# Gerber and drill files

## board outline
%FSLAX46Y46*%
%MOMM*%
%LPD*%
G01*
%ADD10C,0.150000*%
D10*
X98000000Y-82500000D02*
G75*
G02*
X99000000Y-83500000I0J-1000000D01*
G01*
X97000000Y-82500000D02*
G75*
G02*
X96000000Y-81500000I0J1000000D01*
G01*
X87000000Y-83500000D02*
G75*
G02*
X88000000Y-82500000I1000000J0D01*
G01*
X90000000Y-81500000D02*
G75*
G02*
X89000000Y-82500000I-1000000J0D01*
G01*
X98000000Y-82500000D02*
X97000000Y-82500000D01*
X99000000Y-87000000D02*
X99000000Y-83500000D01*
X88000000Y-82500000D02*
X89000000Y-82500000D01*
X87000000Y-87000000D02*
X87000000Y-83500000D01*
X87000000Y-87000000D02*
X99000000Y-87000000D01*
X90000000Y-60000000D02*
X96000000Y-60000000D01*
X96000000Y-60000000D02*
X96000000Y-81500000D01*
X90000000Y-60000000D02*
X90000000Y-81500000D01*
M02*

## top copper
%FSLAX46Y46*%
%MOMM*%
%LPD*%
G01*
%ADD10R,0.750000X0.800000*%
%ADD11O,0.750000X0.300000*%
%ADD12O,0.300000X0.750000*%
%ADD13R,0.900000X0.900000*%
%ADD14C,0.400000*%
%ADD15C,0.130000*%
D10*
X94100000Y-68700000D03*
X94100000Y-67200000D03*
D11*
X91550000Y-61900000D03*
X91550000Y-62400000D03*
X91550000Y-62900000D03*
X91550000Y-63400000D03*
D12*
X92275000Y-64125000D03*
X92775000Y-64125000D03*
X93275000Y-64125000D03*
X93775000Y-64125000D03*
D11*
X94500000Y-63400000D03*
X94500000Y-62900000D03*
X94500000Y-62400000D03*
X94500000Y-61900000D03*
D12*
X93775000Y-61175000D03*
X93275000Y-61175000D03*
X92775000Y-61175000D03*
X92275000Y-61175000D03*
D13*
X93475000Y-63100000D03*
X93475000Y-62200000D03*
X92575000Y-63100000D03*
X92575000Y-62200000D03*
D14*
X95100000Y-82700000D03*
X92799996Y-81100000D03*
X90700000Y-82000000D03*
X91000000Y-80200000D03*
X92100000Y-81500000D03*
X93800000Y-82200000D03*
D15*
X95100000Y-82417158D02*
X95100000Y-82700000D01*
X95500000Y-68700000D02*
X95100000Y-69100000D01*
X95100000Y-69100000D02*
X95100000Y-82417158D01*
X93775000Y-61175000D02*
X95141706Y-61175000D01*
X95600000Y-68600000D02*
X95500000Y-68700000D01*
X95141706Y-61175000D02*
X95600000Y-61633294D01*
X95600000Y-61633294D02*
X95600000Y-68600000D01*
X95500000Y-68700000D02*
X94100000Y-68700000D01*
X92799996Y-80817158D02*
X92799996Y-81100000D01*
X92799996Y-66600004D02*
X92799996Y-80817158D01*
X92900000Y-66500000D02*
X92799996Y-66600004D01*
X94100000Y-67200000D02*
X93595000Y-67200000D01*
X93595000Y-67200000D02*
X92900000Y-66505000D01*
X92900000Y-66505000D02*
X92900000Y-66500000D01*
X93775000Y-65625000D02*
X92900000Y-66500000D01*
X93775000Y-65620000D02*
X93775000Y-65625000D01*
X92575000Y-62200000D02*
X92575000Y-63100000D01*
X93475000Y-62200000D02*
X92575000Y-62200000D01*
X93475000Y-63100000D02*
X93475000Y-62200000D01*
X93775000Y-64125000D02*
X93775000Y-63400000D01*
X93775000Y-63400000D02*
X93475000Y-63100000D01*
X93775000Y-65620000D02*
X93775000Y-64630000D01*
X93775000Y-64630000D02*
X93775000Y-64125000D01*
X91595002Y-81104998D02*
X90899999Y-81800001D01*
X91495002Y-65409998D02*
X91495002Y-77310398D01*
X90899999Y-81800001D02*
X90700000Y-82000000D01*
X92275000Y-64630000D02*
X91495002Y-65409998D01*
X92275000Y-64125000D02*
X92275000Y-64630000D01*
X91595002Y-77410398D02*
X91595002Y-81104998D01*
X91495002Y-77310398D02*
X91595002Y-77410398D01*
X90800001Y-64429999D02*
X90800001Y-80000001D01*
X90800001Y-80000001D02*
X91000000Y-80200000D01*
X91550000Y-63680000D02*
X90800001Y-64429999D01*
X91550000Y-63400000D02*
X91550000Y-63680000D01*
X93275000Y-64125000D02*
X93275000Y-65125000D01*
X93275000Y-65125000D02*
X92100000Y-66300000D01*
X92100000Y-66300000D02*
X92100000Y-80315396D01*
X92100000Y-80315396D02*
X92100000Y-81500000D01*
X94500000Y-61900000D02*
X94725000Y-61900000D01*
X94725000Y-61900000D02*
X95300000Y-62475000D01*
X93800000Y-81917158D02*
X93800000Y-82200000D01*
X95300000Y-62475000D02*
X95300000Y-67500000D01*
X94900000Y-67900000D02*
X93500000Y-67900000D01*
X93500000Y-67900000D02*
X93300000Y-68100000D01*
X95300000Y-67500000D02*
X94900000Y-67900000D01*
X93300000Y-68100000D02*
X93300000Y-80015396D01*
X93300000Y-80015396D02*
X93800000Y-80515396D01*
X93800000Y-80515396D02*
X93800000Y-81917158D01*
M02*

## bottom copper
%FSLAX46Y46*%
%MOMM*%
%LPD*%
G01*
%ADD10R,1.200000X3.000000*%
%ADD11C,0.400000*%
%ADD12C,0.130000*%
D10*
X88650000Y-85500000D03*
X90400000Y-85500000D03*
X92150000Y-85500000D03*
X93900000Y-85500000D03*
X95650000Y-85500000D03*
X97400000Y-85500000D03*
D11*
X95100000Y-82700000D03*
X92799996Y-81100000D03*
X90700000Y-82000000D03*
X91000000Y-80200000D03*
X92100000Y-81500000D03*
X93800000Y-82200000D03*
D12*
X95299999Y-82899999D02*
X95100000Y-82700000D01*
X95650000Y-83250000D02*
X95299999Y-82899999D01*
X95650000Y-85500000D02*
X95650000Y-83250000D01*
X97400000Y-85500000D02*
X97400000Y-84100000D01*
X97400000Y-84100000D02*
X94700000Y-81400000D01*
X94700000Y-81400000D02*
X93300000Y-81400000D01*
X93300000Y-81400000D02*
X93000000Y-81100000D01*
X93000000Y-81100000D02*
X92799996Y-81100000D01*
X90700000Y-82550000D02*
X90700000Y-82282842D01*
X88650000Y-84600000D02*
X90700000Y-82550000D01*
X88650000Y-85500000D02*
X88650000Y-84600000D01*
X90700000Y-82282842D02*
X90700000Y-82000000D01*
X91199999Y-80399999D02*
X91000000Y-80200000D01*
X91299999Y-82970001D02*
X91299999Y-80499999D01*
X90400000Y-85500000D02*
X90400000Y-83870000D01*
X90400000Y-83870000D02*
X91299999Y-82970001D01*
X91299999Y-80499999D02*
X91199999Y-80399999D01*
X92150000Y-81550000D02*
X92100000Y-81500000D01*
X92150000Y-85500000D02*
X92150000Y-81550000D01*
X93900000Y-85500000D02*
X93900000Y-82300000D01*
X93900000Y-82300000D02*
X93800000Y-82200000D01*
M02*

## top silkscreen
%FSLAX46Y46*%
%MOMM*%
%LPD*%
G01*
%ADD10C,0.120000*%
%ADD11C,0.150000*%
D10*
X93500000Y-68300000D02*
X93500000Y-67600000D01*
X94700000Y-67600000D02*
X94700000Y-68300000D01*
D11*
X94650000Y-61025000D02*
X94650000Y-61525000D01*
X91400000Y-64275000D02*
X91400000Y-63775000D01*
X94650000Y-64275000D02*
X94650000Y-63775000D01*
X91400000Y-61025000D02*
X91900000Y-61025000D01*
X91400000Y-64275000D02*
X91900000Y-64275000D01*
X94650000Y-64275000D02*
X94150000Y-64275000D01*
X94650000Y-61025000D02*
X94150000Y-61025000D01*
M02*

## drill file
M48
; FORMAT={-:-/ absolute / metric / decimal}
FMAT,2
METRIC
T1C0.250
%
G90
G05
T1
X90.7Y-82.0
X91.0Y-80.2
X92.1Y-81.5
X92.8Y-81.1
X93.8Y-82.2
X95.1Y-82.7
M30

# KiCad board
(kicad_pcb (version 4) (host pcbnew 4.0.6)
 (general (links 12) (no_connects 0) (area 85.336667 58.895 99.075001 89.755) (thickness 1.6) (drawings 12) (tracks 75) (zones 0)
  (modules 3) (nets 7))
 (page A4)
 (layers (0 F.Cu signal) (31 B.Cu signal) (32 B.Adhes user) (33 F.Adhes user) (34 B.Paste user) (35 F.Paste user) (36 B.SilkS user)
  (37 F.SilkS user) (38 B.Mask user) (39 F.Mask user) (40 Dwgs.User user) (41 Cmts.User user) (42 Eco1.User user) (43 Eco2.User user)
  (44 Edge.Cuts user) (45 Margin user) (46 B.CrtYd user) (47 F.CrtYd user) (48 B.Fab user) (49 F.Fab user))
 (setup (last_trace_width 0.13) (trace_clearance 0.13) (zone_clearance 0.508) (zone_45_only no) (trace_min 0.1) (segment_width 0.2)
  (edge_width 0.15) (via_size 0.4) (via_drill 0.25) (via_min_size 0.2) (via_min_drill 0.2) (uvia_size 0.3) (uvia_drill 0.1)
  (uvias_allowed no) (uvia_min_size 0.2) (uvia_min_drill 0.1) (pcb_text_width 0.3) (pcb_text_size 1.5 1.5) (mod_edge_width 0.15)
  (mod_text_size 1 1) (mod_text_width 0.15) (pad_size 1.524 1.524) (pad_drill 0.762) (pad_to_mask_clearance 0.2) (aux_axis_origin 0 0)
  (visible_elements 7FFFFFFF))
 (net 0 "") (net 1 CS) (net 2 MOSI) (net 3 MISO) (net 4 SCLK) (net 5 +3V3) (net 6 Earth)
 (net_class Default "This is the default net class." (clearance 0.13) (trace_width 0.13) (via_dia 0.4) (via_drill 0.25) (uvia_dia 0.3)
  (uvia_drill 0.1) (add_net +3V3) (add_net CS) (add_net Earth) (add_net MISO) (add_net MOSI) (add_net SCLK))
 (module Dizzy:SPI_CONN (layer B.Cu) (at 90.3 88.25)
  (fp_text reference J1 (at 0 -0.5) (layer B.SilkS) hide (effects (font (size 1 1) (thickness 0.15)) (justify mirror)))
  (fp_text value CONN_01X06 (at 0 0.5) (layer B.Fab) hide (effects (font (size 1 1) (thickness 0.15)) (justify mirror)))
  (pad 1 smd rect (at -1.65 -2.75) (size 1.2 3) (layers B.Cu B.Paste B.Mask) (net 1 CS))
  (pad 2 smd rect (at 0.1 -2.75) (size 1.2 3) (layers B.Cu B.Paste B.Mask) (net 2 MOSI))
  (pad 3 smd rect (at 1.85 -2.75) (size 1.2 3) (layers B.Cu B.Paste B.Mask) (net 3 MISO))
  (pad 4 smd rect (at 3.6 -2.75) (size 1.2 3) (layers B.Cu B.Paste B.Mask) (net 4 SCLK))
  (pad 5 smd rect (at 5.35 -2.75) (size 1.2 3) (layers B.Cu B.Paste B.Mask) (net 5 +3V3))
  (pad 6 smd rect (at 7.1 -2.75) (size 1.2 3) (layers B.Cu B.Paste B.Mask) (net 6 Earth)))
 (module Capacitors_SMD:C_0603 (layer F.Cu) (at 94.1 67.95 270)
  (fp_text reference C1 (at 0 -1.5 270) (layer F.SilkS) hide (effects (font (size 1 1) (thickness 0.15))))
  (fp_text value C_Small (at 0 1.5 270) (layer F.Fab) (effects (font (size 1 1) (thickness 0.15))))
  (fp_line (start 0.35 0.6) (end -0.35 0.6) (layer F.SilkS) (width 0.12))
  (fp_line (start -0.35 -0.6) (end 0.35 -0.6) (layer F.SilkS) (width 0.12))
  (pad 2 smd rect (at 0.75 0 270) (size 0.8 0.75) (layers F.Cu F.Paste F.Mask) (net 5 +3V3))
  (pad 1 smd rect (at -0.75 0 270) (size 0.8 0.75) (layers F.Cu F.Paste F.Mask) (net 6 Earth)))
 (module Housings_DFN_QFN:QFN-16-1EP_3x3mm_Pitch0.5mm (layer F.Cu) (at 93.025 62.65)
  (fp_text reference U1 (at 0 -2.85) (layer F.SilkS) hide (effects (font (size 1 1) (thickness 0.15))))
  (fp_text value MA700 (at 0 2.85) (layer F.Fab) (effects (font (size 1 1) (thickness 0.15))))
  (fp_line (start 1.625 -1.625) (end 1.625 -1.125) (layer F.SilkS) (width 0.15))
  (fp_line (start -1.625 1.625) (end -1.625 1.125) (layer F.SilkS) (width 0.15))
  (fp_line (start 1.625 1.625) (end 1.625 1.125) (layer F.SilkS) (width 0.15))
  (fp_line (start -1.625 -1.625) (end -1.125 -1.625) (layer F.SilkS) (width 0.15))
  (fp_line (start -1.625 1.625) (end -1.125 1.625) (layer F.SilkS) (width 0.15))
  (fp_line (start 1.625 1.625) (end 1.125 1.625) (layer F.SilkS) (width 0.15))
  (fp_line (start 1.625 -1.625) (end 1.125 -1.625) (layer F.SilkS) (width 0.15))
  (pad 1 smd oval (at -1.475 -0.75) (size 0.75 0.3) (layers F.Cu F.Paste F.Mask))
  (pad 2 smd oval (at -1.475 -0.25) (size 0.75 0.3) (layers F.Cu F.Paste F.Mask))
  (pad 3 smd oval (at -1.475 0.25) (size 0.75 0.3) (layers F.Cu F.Paste F.Mask))
  (pad 4 smd oval (at -1.475 0.75) (size 0.75 0.3) (layers F.Cu F.Paste F.Mask) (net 2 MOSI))
  (pad 5 smd oval (at -0.75 1.475 90) (size 0.75 0.3) (layers F.Cu F.Paste F.Mask) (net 1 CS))
  (pad 6 smd oval (at -0.25 1.475 90) (size 0.75 0.3) (layers F.Cu F.Paste F.Mask))
  (pad 7 smd oval (at 0.25 1.475 90) (size 0.75 0.3) (layers F.Cu F.Paste F.Mask) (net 3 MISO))
  (pad 8 smd oval (at 0.75 1.475 90) (size 0.75 0.3) (layers F.Cu F.Paste F.Mask) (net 6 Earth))
  (pad 9 smd oval (at 1.475 0.75) (size 0.75 0.3) (layers F.Cu F.Paste F.Mask))
  (pad 10 smd oval (at 1.475 0.25) (size 0.75 0.3) (layers F.Cu F.Paste F.Mask))
  (pad 11 smd oval (at 1.475 -0.25) (size 0.75 0.3) (layers F.Cu F.Paste F.Mask))
  (pad 12 smd oval (at 1.475 -0.75) (size 0.75 0.3) (layers F.Cu F.Paste F.Mask) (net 4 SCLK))
  (pad 13 smd oval (at 0.75 -1.475 90) (size 0.75 0.3) (layers F.Cu F.Paste F.Mask) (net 5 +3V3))
  (pad 14 smd oval (at 0.25 -1.475 90) (size 0.75 0.3) (layers F.Cu F.Paste F.Mask))
  (pad 15 smd oval (at -0.25 -1.475 90) (size 0.75 0.3) (layers F.Cu F.Paste F.Mask))
  (pad 16 smd oval (at -0.75 -1.475 90) (size 0.75 0.3) (layers F.Cu F.Paste F.Mask))
  (pad 17 smd rect (at 0.45 0.45) (size 0.9 0.9) (layers F.Cu F.Paste F.Mask) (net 6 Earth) (solder_paste_margin_ratio -0.2))
  (pad 17 smd rect (at 0.45 -0.45) (size 0.9 0.9) (layers F.Cu F.Paste F.Mask) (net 6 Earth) (solder_paste_margin_ratio -0.2))
  (pad 17 smd rect (at -0.45 0.45) (size 0.9 0.9) (layers F.Cu F.Paste F.Mask) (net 6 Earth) (solder_paste_margin_ratio -0.2))
  (pad 17 smd rect (at -0.45 -0.45) (size 0.9 0.9) (layers F.Cu F.Paste F.Mask) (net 6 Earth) (solder_paste_margin_ratio -0.2)))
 (gr_arc (start 98 83.5) (end 98 82.5) (angle 90) (layer Edge.Cuts) (width 0.15))
 (gr_arc (start 97 81.5) (end 97 82.5) (angle 90) (layer Edge.Cuts) (width 0.15))
 (gr_arc (start 88 83.5) (end 87 83.5) (angle 90) (layer Edge.Cuts) (width 0.15))
 (gr_arc (start 89 81.5) (end 90 81.5) (angle 90) (layer Edge.Cuts) (width 0.15))
 (gr_line (start 98 82.5) (end 97 82.5) (layer Edge.Cuts) (width 0.15))
 (gr_line (start 99 87) (end 99 83.5) (layer Edge.Cuts) (width 0.15))
 (gr_line (start 88 82.5) (end 89 82.5) (layer Edge.Cuts) (width 0.15))
 (gr_line (start 87 87) (end 87 83.5) (layer Edge.Cuts) (width 0.15))
 (gr_line (start 87 87) (end 99 87) (layer Edge.Cuts) (width 0.15))
 (gr_line (start 90 60) (end 96 60) (layer Edge.Cuts) (width 0.15))
 (gr_line (start 96 60) (end 96 81.5) (layer Edge.Cuts) (width 0.15))
 (gr_line (start 90 60) (end 90 81.5) (layer Edge.Cuts) (width 0.15))
 (segment (start 95.299999 82.899999) (end 95.1 82.7) (width 0.13) (layer B.Cu) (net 5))
 (segment (start 95.65 83.25) (end 95.299999 82.899999) (width 0.13) (layer B.Cu) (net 5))
 (segment (start 95.65 85.5) (end 95.65 83.25) (width 0.13) (layer B.Cu) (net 5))
 (segment (start 95.1 82.417158) (end 95.1 82.7) (width 0.13) (layer F.Cu) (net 5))
 (segment (start 95.5 68.7) (end 95.1 69.1) (width 0.13) (layer F.Cu) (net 5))
 (segment (start 95.1 69.1) (end 95.1 82.417158) (width 0.13) (layer F.Cu) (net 5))
 (via (at 95.1 82.7) (size 0.4) (drill 0.25) (layers F.Cu B.Cu) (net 5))
 (segment (start 93.775 61.175) (end 95.141706 61.175) (width 0.13) (layer F.Cu) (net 5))
 (segment (start 95.6 68.6) (end 95.5 68.7) (width 0.13) (layer F.Cu) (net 5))
 (segment (start 95.141706 61.175) (end 95.6 61.633294) (width 0.13) (layer F.Cu) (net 5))
 (segment (start 95.6 61.633294) (end 95.6 68.6) (width 0.13) (layer F.Cu) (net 5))
 (segment (start 95.5 68.7) (end 94.1 68.7) (width 0.13) (layer F.Cu) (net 5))
 (segment (start 97.4 85.5) (end 97.4 84.1) (width 0.13) (layer B.Cu) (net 6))
 (segment (start 97.4 84.1) (end 94.7 81.4) (width 0.13) (layer B.Cu) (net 6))
 (segment (start 94.7 81.4) (end 93.3 81.4) (width 0.13) (layer B.Cu) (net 6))
 (segment (start 93.3 81.4) (end 93 81.1) (width 0.13) (layer B.Cu) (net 6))
 (segment (start 93 81.1) (end 92.799996 81.1) (width 0.13) (layer B.Cu) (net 6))
 (segment (start 92.799996 80.817158) (end 92.799996 81.1) (width 0.13) (layer F.Cu) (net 6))
 (segment (start 92.799996 66.600004) (end 92.799996 80.817158) (width 0.13) (layer F.Cu) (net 6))
 (segment (start 92.9 66.5) (end 92.799996 66.600004) (width 0.13) (layer F.Cu) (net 6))
 (via (at 92.799996 81.1) (size 0.4) (drill 0.25) (layers F.Cu B.Cu) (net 6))
 (segment (start 94.1 67.2) (end 93.595 67.2) (width 0.13) (layer F.Cu) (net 6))
 (segment (start 93.595 67.2) (end 92.9 66.505) (width 0.13) (layer F.Cu) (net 6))
 (segment (start 92.9 66.505) (end 92.9 66.5) (width 0.13) (layer F.Cu) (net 6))
 (segment (start 93.775 65.625) (end 92.9 66.5) (width 0.13) (layer F.Cu) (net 6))
 (segment (start 93.775 65.62) (end 93.775 65.625) (width 0.13) (layer F.Cu) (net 6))
 (segment (start 92.575 62.2) (end 92.575 63.1) (width 0.13) (layer F.Cu) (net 6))
 (segment (start 93.475 62.2) (end 92.575 62.2) (width 0.13) (layer F.Cu) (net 6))
 (segment (start 93.475 63.1) (end 93.475 62.2) (width 0.13) (layer F.Cu) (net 6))
 (segment (start 93.775 64.125) (end 93.775 63.4) (width 0.13) (layer F.Cu) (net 6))
 (segment (start 93.775 63.4) (end 93.475 63.1) (width 0.13) (layer F.Cu) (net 6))
 (segment (start 93.775 65.62) (end 93.775 64.63) (width 0.13) (layer F.Cu) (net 6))
 (segment (start 93.775 64.63) (end 93.775 64.125) (width 0.13) (layer F.Cu) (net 6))
 (segment (start 91.595002 81.104998) (end 90.899999 81.800001) (width 0.13) (layer F.Cu) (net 1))
 (segment (start 91.495002 65.409998) (end 91.495002 77.310398) (width 0.13) (layer F.Cu) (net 1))
 (segment (start 90.899999 81.800001) (end 90.7 82) (width 0.13) (layer F.Cu) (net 1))
 (segment (start 92.275 64.63) (end 91.495002 65.409998) (width 0.13) (layer F.Cu) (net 1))
 (segment (start 92.275 64.125) (end 92.275 64.63) (width 0.13) (layer F.Cu) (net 1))
 (segment (start 91.595002 77.410398) (end 91.595002 81.104998) (width 0.13) (layer F.Cu) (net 1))
 (segment (start 91.495002 77.310398) (end 91.595002 77.410398) (width 0.13) (layer F.Cu) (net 1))
 (segment (start 90.7 82.55) (end 90.7 82.282842) (width 0.13) (layer B.Cu) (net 1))
 (segment (start 88.65 84.6) (end 90.7 82.55) (width 0.13) (layer B.Cu) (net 1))
 (segment (start 88.65 85.5) (end 88.65 84.6) (width 0.13) (layer B.Cu) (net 1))
 (segment (start 90.7 82.282842) (end 90.7 82) (width 0.13) (layer B.Cu) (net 1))
 (via (at 90.7 82) (size 0.4) (drill 0.25) (layers F.Cu B.Cu) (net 1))
 (segment (start 91.199999 80.399999) (end 91 80.2) (width 0.13) (layer B.Cu) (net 2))
 (segment (start 91.299999 82.970001) (end 91.299999 80.499999) (width 0.13) (layer B.Cu) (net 2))
 (segment (start 90.4 85.5) (end 90.4 83.87) (width 0.13) (layer B.Cu) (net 2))
 (segment (start 90.4 83.87) (end 91.299999 82.970001) (width 0.13) (layer B.Cu) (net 2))
 (segment (start 90.800001 64.429999) (end 90.800001 80.000001) (width 0.13) (layer F.Cu) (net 2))
 (segment (start 91.299999 80.499999) (end 91.199999 80.399999) (width 0.13) (layer B.Cu) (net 2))
 (segment (start 90.800001 80.000001) (end 91 80.2) (width 0.13) (layer F.Cu) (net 2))
 (segment (start 91.55 63.68) (end 90.800001 64.429999) (width 0.13) (layer F.Cu) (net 2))
 (segment (start 91.55 63.4) (end 91.55 63.68) (width 0.13) (layer F.Cu) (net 2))
 (via (at 91 80.2) (size 0.4) (drill 0.25) (layers F.Cu B.Cu) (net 2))
 (segment (start 93.275 64.125) (end 93.275 65.125) (width 0.13) (layer F.Cu) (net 3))
 (segment (start 93.275 65.125) (end 92.1 66.3) (width 0.13) (layer F.Cu) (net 3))
 (segment (start 92.1 66.3) (end 92.1 80.315396) (width 0.13) (layer F.Cu) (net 3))
 (segment (start 92.1 80.315396) (end 92.1 81.5) (width 0.13) (layer F.Cu) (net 3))
 (segment (start 92.15 81.55) (end 92.1 81.5) (width 0.13) (layer B.Cu) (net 3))
 (segment (start 92.15 85.5) (end 92.15 81.55) (width 0.13) (layer B.Cu) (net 3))
 (via (at 92.1 81.5) (size 0.4) (drill 0.25) (layers F.Cu B.Cu) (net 3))
 (segment (start 94.5 61.9) (end 94.725 61.9) (width 0.13) (layer F.Cu) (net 4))
 (segment (start 94.725 61.9) (end 95.3 62.475) (width 0.13) (layer F.Cu) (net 4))
 (segment (start 93.8 81.917158) (end 93.8 82.2) (width 0.13) (layer F.Cu) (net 4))
 (segment (start 95.3 62.475) (end 95.3 67.5) (width 0.13) (layer F.Cu) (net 4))
 (segment (start 94.9 67.9) (end 93.5 67.9) (width 0.13) (layer F.Cu) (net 4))
 (segment (start 93.5 67.9) (end 93.3 68.1) (width 0.13) (layer F.Cu) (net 4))
 (segment (start 95.3 67.5) (end 94.9 67.9) (width 0.13) (layer F.Cu) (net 4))
 (segment (start 93.3 68.1) (end 93.3 80.015396) (width 0.13) (layer F.Cu) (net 4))
 (segment (start 93.3 80.015396) (end 93.8 80.515396) (width 0.13) (layer F.Cu) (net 4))
 (segment (start 93.8 80.515396) (end 93.8 81.917158) (width 0.13) (layer F.Cu) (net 4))
 (segment (start 93.9 85.5) (end 93.9 82.3) (width 0.13) (layer B.Cu) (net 4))
 (segment (start 93.9 82.3) (end 93.8 82.2) (width 0.13) (layer B.Cu) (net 4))
 (via (at 93.8 82.2) (size 0.4) (drill 0.25) (layers F.Cu B.Cu) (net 4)))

